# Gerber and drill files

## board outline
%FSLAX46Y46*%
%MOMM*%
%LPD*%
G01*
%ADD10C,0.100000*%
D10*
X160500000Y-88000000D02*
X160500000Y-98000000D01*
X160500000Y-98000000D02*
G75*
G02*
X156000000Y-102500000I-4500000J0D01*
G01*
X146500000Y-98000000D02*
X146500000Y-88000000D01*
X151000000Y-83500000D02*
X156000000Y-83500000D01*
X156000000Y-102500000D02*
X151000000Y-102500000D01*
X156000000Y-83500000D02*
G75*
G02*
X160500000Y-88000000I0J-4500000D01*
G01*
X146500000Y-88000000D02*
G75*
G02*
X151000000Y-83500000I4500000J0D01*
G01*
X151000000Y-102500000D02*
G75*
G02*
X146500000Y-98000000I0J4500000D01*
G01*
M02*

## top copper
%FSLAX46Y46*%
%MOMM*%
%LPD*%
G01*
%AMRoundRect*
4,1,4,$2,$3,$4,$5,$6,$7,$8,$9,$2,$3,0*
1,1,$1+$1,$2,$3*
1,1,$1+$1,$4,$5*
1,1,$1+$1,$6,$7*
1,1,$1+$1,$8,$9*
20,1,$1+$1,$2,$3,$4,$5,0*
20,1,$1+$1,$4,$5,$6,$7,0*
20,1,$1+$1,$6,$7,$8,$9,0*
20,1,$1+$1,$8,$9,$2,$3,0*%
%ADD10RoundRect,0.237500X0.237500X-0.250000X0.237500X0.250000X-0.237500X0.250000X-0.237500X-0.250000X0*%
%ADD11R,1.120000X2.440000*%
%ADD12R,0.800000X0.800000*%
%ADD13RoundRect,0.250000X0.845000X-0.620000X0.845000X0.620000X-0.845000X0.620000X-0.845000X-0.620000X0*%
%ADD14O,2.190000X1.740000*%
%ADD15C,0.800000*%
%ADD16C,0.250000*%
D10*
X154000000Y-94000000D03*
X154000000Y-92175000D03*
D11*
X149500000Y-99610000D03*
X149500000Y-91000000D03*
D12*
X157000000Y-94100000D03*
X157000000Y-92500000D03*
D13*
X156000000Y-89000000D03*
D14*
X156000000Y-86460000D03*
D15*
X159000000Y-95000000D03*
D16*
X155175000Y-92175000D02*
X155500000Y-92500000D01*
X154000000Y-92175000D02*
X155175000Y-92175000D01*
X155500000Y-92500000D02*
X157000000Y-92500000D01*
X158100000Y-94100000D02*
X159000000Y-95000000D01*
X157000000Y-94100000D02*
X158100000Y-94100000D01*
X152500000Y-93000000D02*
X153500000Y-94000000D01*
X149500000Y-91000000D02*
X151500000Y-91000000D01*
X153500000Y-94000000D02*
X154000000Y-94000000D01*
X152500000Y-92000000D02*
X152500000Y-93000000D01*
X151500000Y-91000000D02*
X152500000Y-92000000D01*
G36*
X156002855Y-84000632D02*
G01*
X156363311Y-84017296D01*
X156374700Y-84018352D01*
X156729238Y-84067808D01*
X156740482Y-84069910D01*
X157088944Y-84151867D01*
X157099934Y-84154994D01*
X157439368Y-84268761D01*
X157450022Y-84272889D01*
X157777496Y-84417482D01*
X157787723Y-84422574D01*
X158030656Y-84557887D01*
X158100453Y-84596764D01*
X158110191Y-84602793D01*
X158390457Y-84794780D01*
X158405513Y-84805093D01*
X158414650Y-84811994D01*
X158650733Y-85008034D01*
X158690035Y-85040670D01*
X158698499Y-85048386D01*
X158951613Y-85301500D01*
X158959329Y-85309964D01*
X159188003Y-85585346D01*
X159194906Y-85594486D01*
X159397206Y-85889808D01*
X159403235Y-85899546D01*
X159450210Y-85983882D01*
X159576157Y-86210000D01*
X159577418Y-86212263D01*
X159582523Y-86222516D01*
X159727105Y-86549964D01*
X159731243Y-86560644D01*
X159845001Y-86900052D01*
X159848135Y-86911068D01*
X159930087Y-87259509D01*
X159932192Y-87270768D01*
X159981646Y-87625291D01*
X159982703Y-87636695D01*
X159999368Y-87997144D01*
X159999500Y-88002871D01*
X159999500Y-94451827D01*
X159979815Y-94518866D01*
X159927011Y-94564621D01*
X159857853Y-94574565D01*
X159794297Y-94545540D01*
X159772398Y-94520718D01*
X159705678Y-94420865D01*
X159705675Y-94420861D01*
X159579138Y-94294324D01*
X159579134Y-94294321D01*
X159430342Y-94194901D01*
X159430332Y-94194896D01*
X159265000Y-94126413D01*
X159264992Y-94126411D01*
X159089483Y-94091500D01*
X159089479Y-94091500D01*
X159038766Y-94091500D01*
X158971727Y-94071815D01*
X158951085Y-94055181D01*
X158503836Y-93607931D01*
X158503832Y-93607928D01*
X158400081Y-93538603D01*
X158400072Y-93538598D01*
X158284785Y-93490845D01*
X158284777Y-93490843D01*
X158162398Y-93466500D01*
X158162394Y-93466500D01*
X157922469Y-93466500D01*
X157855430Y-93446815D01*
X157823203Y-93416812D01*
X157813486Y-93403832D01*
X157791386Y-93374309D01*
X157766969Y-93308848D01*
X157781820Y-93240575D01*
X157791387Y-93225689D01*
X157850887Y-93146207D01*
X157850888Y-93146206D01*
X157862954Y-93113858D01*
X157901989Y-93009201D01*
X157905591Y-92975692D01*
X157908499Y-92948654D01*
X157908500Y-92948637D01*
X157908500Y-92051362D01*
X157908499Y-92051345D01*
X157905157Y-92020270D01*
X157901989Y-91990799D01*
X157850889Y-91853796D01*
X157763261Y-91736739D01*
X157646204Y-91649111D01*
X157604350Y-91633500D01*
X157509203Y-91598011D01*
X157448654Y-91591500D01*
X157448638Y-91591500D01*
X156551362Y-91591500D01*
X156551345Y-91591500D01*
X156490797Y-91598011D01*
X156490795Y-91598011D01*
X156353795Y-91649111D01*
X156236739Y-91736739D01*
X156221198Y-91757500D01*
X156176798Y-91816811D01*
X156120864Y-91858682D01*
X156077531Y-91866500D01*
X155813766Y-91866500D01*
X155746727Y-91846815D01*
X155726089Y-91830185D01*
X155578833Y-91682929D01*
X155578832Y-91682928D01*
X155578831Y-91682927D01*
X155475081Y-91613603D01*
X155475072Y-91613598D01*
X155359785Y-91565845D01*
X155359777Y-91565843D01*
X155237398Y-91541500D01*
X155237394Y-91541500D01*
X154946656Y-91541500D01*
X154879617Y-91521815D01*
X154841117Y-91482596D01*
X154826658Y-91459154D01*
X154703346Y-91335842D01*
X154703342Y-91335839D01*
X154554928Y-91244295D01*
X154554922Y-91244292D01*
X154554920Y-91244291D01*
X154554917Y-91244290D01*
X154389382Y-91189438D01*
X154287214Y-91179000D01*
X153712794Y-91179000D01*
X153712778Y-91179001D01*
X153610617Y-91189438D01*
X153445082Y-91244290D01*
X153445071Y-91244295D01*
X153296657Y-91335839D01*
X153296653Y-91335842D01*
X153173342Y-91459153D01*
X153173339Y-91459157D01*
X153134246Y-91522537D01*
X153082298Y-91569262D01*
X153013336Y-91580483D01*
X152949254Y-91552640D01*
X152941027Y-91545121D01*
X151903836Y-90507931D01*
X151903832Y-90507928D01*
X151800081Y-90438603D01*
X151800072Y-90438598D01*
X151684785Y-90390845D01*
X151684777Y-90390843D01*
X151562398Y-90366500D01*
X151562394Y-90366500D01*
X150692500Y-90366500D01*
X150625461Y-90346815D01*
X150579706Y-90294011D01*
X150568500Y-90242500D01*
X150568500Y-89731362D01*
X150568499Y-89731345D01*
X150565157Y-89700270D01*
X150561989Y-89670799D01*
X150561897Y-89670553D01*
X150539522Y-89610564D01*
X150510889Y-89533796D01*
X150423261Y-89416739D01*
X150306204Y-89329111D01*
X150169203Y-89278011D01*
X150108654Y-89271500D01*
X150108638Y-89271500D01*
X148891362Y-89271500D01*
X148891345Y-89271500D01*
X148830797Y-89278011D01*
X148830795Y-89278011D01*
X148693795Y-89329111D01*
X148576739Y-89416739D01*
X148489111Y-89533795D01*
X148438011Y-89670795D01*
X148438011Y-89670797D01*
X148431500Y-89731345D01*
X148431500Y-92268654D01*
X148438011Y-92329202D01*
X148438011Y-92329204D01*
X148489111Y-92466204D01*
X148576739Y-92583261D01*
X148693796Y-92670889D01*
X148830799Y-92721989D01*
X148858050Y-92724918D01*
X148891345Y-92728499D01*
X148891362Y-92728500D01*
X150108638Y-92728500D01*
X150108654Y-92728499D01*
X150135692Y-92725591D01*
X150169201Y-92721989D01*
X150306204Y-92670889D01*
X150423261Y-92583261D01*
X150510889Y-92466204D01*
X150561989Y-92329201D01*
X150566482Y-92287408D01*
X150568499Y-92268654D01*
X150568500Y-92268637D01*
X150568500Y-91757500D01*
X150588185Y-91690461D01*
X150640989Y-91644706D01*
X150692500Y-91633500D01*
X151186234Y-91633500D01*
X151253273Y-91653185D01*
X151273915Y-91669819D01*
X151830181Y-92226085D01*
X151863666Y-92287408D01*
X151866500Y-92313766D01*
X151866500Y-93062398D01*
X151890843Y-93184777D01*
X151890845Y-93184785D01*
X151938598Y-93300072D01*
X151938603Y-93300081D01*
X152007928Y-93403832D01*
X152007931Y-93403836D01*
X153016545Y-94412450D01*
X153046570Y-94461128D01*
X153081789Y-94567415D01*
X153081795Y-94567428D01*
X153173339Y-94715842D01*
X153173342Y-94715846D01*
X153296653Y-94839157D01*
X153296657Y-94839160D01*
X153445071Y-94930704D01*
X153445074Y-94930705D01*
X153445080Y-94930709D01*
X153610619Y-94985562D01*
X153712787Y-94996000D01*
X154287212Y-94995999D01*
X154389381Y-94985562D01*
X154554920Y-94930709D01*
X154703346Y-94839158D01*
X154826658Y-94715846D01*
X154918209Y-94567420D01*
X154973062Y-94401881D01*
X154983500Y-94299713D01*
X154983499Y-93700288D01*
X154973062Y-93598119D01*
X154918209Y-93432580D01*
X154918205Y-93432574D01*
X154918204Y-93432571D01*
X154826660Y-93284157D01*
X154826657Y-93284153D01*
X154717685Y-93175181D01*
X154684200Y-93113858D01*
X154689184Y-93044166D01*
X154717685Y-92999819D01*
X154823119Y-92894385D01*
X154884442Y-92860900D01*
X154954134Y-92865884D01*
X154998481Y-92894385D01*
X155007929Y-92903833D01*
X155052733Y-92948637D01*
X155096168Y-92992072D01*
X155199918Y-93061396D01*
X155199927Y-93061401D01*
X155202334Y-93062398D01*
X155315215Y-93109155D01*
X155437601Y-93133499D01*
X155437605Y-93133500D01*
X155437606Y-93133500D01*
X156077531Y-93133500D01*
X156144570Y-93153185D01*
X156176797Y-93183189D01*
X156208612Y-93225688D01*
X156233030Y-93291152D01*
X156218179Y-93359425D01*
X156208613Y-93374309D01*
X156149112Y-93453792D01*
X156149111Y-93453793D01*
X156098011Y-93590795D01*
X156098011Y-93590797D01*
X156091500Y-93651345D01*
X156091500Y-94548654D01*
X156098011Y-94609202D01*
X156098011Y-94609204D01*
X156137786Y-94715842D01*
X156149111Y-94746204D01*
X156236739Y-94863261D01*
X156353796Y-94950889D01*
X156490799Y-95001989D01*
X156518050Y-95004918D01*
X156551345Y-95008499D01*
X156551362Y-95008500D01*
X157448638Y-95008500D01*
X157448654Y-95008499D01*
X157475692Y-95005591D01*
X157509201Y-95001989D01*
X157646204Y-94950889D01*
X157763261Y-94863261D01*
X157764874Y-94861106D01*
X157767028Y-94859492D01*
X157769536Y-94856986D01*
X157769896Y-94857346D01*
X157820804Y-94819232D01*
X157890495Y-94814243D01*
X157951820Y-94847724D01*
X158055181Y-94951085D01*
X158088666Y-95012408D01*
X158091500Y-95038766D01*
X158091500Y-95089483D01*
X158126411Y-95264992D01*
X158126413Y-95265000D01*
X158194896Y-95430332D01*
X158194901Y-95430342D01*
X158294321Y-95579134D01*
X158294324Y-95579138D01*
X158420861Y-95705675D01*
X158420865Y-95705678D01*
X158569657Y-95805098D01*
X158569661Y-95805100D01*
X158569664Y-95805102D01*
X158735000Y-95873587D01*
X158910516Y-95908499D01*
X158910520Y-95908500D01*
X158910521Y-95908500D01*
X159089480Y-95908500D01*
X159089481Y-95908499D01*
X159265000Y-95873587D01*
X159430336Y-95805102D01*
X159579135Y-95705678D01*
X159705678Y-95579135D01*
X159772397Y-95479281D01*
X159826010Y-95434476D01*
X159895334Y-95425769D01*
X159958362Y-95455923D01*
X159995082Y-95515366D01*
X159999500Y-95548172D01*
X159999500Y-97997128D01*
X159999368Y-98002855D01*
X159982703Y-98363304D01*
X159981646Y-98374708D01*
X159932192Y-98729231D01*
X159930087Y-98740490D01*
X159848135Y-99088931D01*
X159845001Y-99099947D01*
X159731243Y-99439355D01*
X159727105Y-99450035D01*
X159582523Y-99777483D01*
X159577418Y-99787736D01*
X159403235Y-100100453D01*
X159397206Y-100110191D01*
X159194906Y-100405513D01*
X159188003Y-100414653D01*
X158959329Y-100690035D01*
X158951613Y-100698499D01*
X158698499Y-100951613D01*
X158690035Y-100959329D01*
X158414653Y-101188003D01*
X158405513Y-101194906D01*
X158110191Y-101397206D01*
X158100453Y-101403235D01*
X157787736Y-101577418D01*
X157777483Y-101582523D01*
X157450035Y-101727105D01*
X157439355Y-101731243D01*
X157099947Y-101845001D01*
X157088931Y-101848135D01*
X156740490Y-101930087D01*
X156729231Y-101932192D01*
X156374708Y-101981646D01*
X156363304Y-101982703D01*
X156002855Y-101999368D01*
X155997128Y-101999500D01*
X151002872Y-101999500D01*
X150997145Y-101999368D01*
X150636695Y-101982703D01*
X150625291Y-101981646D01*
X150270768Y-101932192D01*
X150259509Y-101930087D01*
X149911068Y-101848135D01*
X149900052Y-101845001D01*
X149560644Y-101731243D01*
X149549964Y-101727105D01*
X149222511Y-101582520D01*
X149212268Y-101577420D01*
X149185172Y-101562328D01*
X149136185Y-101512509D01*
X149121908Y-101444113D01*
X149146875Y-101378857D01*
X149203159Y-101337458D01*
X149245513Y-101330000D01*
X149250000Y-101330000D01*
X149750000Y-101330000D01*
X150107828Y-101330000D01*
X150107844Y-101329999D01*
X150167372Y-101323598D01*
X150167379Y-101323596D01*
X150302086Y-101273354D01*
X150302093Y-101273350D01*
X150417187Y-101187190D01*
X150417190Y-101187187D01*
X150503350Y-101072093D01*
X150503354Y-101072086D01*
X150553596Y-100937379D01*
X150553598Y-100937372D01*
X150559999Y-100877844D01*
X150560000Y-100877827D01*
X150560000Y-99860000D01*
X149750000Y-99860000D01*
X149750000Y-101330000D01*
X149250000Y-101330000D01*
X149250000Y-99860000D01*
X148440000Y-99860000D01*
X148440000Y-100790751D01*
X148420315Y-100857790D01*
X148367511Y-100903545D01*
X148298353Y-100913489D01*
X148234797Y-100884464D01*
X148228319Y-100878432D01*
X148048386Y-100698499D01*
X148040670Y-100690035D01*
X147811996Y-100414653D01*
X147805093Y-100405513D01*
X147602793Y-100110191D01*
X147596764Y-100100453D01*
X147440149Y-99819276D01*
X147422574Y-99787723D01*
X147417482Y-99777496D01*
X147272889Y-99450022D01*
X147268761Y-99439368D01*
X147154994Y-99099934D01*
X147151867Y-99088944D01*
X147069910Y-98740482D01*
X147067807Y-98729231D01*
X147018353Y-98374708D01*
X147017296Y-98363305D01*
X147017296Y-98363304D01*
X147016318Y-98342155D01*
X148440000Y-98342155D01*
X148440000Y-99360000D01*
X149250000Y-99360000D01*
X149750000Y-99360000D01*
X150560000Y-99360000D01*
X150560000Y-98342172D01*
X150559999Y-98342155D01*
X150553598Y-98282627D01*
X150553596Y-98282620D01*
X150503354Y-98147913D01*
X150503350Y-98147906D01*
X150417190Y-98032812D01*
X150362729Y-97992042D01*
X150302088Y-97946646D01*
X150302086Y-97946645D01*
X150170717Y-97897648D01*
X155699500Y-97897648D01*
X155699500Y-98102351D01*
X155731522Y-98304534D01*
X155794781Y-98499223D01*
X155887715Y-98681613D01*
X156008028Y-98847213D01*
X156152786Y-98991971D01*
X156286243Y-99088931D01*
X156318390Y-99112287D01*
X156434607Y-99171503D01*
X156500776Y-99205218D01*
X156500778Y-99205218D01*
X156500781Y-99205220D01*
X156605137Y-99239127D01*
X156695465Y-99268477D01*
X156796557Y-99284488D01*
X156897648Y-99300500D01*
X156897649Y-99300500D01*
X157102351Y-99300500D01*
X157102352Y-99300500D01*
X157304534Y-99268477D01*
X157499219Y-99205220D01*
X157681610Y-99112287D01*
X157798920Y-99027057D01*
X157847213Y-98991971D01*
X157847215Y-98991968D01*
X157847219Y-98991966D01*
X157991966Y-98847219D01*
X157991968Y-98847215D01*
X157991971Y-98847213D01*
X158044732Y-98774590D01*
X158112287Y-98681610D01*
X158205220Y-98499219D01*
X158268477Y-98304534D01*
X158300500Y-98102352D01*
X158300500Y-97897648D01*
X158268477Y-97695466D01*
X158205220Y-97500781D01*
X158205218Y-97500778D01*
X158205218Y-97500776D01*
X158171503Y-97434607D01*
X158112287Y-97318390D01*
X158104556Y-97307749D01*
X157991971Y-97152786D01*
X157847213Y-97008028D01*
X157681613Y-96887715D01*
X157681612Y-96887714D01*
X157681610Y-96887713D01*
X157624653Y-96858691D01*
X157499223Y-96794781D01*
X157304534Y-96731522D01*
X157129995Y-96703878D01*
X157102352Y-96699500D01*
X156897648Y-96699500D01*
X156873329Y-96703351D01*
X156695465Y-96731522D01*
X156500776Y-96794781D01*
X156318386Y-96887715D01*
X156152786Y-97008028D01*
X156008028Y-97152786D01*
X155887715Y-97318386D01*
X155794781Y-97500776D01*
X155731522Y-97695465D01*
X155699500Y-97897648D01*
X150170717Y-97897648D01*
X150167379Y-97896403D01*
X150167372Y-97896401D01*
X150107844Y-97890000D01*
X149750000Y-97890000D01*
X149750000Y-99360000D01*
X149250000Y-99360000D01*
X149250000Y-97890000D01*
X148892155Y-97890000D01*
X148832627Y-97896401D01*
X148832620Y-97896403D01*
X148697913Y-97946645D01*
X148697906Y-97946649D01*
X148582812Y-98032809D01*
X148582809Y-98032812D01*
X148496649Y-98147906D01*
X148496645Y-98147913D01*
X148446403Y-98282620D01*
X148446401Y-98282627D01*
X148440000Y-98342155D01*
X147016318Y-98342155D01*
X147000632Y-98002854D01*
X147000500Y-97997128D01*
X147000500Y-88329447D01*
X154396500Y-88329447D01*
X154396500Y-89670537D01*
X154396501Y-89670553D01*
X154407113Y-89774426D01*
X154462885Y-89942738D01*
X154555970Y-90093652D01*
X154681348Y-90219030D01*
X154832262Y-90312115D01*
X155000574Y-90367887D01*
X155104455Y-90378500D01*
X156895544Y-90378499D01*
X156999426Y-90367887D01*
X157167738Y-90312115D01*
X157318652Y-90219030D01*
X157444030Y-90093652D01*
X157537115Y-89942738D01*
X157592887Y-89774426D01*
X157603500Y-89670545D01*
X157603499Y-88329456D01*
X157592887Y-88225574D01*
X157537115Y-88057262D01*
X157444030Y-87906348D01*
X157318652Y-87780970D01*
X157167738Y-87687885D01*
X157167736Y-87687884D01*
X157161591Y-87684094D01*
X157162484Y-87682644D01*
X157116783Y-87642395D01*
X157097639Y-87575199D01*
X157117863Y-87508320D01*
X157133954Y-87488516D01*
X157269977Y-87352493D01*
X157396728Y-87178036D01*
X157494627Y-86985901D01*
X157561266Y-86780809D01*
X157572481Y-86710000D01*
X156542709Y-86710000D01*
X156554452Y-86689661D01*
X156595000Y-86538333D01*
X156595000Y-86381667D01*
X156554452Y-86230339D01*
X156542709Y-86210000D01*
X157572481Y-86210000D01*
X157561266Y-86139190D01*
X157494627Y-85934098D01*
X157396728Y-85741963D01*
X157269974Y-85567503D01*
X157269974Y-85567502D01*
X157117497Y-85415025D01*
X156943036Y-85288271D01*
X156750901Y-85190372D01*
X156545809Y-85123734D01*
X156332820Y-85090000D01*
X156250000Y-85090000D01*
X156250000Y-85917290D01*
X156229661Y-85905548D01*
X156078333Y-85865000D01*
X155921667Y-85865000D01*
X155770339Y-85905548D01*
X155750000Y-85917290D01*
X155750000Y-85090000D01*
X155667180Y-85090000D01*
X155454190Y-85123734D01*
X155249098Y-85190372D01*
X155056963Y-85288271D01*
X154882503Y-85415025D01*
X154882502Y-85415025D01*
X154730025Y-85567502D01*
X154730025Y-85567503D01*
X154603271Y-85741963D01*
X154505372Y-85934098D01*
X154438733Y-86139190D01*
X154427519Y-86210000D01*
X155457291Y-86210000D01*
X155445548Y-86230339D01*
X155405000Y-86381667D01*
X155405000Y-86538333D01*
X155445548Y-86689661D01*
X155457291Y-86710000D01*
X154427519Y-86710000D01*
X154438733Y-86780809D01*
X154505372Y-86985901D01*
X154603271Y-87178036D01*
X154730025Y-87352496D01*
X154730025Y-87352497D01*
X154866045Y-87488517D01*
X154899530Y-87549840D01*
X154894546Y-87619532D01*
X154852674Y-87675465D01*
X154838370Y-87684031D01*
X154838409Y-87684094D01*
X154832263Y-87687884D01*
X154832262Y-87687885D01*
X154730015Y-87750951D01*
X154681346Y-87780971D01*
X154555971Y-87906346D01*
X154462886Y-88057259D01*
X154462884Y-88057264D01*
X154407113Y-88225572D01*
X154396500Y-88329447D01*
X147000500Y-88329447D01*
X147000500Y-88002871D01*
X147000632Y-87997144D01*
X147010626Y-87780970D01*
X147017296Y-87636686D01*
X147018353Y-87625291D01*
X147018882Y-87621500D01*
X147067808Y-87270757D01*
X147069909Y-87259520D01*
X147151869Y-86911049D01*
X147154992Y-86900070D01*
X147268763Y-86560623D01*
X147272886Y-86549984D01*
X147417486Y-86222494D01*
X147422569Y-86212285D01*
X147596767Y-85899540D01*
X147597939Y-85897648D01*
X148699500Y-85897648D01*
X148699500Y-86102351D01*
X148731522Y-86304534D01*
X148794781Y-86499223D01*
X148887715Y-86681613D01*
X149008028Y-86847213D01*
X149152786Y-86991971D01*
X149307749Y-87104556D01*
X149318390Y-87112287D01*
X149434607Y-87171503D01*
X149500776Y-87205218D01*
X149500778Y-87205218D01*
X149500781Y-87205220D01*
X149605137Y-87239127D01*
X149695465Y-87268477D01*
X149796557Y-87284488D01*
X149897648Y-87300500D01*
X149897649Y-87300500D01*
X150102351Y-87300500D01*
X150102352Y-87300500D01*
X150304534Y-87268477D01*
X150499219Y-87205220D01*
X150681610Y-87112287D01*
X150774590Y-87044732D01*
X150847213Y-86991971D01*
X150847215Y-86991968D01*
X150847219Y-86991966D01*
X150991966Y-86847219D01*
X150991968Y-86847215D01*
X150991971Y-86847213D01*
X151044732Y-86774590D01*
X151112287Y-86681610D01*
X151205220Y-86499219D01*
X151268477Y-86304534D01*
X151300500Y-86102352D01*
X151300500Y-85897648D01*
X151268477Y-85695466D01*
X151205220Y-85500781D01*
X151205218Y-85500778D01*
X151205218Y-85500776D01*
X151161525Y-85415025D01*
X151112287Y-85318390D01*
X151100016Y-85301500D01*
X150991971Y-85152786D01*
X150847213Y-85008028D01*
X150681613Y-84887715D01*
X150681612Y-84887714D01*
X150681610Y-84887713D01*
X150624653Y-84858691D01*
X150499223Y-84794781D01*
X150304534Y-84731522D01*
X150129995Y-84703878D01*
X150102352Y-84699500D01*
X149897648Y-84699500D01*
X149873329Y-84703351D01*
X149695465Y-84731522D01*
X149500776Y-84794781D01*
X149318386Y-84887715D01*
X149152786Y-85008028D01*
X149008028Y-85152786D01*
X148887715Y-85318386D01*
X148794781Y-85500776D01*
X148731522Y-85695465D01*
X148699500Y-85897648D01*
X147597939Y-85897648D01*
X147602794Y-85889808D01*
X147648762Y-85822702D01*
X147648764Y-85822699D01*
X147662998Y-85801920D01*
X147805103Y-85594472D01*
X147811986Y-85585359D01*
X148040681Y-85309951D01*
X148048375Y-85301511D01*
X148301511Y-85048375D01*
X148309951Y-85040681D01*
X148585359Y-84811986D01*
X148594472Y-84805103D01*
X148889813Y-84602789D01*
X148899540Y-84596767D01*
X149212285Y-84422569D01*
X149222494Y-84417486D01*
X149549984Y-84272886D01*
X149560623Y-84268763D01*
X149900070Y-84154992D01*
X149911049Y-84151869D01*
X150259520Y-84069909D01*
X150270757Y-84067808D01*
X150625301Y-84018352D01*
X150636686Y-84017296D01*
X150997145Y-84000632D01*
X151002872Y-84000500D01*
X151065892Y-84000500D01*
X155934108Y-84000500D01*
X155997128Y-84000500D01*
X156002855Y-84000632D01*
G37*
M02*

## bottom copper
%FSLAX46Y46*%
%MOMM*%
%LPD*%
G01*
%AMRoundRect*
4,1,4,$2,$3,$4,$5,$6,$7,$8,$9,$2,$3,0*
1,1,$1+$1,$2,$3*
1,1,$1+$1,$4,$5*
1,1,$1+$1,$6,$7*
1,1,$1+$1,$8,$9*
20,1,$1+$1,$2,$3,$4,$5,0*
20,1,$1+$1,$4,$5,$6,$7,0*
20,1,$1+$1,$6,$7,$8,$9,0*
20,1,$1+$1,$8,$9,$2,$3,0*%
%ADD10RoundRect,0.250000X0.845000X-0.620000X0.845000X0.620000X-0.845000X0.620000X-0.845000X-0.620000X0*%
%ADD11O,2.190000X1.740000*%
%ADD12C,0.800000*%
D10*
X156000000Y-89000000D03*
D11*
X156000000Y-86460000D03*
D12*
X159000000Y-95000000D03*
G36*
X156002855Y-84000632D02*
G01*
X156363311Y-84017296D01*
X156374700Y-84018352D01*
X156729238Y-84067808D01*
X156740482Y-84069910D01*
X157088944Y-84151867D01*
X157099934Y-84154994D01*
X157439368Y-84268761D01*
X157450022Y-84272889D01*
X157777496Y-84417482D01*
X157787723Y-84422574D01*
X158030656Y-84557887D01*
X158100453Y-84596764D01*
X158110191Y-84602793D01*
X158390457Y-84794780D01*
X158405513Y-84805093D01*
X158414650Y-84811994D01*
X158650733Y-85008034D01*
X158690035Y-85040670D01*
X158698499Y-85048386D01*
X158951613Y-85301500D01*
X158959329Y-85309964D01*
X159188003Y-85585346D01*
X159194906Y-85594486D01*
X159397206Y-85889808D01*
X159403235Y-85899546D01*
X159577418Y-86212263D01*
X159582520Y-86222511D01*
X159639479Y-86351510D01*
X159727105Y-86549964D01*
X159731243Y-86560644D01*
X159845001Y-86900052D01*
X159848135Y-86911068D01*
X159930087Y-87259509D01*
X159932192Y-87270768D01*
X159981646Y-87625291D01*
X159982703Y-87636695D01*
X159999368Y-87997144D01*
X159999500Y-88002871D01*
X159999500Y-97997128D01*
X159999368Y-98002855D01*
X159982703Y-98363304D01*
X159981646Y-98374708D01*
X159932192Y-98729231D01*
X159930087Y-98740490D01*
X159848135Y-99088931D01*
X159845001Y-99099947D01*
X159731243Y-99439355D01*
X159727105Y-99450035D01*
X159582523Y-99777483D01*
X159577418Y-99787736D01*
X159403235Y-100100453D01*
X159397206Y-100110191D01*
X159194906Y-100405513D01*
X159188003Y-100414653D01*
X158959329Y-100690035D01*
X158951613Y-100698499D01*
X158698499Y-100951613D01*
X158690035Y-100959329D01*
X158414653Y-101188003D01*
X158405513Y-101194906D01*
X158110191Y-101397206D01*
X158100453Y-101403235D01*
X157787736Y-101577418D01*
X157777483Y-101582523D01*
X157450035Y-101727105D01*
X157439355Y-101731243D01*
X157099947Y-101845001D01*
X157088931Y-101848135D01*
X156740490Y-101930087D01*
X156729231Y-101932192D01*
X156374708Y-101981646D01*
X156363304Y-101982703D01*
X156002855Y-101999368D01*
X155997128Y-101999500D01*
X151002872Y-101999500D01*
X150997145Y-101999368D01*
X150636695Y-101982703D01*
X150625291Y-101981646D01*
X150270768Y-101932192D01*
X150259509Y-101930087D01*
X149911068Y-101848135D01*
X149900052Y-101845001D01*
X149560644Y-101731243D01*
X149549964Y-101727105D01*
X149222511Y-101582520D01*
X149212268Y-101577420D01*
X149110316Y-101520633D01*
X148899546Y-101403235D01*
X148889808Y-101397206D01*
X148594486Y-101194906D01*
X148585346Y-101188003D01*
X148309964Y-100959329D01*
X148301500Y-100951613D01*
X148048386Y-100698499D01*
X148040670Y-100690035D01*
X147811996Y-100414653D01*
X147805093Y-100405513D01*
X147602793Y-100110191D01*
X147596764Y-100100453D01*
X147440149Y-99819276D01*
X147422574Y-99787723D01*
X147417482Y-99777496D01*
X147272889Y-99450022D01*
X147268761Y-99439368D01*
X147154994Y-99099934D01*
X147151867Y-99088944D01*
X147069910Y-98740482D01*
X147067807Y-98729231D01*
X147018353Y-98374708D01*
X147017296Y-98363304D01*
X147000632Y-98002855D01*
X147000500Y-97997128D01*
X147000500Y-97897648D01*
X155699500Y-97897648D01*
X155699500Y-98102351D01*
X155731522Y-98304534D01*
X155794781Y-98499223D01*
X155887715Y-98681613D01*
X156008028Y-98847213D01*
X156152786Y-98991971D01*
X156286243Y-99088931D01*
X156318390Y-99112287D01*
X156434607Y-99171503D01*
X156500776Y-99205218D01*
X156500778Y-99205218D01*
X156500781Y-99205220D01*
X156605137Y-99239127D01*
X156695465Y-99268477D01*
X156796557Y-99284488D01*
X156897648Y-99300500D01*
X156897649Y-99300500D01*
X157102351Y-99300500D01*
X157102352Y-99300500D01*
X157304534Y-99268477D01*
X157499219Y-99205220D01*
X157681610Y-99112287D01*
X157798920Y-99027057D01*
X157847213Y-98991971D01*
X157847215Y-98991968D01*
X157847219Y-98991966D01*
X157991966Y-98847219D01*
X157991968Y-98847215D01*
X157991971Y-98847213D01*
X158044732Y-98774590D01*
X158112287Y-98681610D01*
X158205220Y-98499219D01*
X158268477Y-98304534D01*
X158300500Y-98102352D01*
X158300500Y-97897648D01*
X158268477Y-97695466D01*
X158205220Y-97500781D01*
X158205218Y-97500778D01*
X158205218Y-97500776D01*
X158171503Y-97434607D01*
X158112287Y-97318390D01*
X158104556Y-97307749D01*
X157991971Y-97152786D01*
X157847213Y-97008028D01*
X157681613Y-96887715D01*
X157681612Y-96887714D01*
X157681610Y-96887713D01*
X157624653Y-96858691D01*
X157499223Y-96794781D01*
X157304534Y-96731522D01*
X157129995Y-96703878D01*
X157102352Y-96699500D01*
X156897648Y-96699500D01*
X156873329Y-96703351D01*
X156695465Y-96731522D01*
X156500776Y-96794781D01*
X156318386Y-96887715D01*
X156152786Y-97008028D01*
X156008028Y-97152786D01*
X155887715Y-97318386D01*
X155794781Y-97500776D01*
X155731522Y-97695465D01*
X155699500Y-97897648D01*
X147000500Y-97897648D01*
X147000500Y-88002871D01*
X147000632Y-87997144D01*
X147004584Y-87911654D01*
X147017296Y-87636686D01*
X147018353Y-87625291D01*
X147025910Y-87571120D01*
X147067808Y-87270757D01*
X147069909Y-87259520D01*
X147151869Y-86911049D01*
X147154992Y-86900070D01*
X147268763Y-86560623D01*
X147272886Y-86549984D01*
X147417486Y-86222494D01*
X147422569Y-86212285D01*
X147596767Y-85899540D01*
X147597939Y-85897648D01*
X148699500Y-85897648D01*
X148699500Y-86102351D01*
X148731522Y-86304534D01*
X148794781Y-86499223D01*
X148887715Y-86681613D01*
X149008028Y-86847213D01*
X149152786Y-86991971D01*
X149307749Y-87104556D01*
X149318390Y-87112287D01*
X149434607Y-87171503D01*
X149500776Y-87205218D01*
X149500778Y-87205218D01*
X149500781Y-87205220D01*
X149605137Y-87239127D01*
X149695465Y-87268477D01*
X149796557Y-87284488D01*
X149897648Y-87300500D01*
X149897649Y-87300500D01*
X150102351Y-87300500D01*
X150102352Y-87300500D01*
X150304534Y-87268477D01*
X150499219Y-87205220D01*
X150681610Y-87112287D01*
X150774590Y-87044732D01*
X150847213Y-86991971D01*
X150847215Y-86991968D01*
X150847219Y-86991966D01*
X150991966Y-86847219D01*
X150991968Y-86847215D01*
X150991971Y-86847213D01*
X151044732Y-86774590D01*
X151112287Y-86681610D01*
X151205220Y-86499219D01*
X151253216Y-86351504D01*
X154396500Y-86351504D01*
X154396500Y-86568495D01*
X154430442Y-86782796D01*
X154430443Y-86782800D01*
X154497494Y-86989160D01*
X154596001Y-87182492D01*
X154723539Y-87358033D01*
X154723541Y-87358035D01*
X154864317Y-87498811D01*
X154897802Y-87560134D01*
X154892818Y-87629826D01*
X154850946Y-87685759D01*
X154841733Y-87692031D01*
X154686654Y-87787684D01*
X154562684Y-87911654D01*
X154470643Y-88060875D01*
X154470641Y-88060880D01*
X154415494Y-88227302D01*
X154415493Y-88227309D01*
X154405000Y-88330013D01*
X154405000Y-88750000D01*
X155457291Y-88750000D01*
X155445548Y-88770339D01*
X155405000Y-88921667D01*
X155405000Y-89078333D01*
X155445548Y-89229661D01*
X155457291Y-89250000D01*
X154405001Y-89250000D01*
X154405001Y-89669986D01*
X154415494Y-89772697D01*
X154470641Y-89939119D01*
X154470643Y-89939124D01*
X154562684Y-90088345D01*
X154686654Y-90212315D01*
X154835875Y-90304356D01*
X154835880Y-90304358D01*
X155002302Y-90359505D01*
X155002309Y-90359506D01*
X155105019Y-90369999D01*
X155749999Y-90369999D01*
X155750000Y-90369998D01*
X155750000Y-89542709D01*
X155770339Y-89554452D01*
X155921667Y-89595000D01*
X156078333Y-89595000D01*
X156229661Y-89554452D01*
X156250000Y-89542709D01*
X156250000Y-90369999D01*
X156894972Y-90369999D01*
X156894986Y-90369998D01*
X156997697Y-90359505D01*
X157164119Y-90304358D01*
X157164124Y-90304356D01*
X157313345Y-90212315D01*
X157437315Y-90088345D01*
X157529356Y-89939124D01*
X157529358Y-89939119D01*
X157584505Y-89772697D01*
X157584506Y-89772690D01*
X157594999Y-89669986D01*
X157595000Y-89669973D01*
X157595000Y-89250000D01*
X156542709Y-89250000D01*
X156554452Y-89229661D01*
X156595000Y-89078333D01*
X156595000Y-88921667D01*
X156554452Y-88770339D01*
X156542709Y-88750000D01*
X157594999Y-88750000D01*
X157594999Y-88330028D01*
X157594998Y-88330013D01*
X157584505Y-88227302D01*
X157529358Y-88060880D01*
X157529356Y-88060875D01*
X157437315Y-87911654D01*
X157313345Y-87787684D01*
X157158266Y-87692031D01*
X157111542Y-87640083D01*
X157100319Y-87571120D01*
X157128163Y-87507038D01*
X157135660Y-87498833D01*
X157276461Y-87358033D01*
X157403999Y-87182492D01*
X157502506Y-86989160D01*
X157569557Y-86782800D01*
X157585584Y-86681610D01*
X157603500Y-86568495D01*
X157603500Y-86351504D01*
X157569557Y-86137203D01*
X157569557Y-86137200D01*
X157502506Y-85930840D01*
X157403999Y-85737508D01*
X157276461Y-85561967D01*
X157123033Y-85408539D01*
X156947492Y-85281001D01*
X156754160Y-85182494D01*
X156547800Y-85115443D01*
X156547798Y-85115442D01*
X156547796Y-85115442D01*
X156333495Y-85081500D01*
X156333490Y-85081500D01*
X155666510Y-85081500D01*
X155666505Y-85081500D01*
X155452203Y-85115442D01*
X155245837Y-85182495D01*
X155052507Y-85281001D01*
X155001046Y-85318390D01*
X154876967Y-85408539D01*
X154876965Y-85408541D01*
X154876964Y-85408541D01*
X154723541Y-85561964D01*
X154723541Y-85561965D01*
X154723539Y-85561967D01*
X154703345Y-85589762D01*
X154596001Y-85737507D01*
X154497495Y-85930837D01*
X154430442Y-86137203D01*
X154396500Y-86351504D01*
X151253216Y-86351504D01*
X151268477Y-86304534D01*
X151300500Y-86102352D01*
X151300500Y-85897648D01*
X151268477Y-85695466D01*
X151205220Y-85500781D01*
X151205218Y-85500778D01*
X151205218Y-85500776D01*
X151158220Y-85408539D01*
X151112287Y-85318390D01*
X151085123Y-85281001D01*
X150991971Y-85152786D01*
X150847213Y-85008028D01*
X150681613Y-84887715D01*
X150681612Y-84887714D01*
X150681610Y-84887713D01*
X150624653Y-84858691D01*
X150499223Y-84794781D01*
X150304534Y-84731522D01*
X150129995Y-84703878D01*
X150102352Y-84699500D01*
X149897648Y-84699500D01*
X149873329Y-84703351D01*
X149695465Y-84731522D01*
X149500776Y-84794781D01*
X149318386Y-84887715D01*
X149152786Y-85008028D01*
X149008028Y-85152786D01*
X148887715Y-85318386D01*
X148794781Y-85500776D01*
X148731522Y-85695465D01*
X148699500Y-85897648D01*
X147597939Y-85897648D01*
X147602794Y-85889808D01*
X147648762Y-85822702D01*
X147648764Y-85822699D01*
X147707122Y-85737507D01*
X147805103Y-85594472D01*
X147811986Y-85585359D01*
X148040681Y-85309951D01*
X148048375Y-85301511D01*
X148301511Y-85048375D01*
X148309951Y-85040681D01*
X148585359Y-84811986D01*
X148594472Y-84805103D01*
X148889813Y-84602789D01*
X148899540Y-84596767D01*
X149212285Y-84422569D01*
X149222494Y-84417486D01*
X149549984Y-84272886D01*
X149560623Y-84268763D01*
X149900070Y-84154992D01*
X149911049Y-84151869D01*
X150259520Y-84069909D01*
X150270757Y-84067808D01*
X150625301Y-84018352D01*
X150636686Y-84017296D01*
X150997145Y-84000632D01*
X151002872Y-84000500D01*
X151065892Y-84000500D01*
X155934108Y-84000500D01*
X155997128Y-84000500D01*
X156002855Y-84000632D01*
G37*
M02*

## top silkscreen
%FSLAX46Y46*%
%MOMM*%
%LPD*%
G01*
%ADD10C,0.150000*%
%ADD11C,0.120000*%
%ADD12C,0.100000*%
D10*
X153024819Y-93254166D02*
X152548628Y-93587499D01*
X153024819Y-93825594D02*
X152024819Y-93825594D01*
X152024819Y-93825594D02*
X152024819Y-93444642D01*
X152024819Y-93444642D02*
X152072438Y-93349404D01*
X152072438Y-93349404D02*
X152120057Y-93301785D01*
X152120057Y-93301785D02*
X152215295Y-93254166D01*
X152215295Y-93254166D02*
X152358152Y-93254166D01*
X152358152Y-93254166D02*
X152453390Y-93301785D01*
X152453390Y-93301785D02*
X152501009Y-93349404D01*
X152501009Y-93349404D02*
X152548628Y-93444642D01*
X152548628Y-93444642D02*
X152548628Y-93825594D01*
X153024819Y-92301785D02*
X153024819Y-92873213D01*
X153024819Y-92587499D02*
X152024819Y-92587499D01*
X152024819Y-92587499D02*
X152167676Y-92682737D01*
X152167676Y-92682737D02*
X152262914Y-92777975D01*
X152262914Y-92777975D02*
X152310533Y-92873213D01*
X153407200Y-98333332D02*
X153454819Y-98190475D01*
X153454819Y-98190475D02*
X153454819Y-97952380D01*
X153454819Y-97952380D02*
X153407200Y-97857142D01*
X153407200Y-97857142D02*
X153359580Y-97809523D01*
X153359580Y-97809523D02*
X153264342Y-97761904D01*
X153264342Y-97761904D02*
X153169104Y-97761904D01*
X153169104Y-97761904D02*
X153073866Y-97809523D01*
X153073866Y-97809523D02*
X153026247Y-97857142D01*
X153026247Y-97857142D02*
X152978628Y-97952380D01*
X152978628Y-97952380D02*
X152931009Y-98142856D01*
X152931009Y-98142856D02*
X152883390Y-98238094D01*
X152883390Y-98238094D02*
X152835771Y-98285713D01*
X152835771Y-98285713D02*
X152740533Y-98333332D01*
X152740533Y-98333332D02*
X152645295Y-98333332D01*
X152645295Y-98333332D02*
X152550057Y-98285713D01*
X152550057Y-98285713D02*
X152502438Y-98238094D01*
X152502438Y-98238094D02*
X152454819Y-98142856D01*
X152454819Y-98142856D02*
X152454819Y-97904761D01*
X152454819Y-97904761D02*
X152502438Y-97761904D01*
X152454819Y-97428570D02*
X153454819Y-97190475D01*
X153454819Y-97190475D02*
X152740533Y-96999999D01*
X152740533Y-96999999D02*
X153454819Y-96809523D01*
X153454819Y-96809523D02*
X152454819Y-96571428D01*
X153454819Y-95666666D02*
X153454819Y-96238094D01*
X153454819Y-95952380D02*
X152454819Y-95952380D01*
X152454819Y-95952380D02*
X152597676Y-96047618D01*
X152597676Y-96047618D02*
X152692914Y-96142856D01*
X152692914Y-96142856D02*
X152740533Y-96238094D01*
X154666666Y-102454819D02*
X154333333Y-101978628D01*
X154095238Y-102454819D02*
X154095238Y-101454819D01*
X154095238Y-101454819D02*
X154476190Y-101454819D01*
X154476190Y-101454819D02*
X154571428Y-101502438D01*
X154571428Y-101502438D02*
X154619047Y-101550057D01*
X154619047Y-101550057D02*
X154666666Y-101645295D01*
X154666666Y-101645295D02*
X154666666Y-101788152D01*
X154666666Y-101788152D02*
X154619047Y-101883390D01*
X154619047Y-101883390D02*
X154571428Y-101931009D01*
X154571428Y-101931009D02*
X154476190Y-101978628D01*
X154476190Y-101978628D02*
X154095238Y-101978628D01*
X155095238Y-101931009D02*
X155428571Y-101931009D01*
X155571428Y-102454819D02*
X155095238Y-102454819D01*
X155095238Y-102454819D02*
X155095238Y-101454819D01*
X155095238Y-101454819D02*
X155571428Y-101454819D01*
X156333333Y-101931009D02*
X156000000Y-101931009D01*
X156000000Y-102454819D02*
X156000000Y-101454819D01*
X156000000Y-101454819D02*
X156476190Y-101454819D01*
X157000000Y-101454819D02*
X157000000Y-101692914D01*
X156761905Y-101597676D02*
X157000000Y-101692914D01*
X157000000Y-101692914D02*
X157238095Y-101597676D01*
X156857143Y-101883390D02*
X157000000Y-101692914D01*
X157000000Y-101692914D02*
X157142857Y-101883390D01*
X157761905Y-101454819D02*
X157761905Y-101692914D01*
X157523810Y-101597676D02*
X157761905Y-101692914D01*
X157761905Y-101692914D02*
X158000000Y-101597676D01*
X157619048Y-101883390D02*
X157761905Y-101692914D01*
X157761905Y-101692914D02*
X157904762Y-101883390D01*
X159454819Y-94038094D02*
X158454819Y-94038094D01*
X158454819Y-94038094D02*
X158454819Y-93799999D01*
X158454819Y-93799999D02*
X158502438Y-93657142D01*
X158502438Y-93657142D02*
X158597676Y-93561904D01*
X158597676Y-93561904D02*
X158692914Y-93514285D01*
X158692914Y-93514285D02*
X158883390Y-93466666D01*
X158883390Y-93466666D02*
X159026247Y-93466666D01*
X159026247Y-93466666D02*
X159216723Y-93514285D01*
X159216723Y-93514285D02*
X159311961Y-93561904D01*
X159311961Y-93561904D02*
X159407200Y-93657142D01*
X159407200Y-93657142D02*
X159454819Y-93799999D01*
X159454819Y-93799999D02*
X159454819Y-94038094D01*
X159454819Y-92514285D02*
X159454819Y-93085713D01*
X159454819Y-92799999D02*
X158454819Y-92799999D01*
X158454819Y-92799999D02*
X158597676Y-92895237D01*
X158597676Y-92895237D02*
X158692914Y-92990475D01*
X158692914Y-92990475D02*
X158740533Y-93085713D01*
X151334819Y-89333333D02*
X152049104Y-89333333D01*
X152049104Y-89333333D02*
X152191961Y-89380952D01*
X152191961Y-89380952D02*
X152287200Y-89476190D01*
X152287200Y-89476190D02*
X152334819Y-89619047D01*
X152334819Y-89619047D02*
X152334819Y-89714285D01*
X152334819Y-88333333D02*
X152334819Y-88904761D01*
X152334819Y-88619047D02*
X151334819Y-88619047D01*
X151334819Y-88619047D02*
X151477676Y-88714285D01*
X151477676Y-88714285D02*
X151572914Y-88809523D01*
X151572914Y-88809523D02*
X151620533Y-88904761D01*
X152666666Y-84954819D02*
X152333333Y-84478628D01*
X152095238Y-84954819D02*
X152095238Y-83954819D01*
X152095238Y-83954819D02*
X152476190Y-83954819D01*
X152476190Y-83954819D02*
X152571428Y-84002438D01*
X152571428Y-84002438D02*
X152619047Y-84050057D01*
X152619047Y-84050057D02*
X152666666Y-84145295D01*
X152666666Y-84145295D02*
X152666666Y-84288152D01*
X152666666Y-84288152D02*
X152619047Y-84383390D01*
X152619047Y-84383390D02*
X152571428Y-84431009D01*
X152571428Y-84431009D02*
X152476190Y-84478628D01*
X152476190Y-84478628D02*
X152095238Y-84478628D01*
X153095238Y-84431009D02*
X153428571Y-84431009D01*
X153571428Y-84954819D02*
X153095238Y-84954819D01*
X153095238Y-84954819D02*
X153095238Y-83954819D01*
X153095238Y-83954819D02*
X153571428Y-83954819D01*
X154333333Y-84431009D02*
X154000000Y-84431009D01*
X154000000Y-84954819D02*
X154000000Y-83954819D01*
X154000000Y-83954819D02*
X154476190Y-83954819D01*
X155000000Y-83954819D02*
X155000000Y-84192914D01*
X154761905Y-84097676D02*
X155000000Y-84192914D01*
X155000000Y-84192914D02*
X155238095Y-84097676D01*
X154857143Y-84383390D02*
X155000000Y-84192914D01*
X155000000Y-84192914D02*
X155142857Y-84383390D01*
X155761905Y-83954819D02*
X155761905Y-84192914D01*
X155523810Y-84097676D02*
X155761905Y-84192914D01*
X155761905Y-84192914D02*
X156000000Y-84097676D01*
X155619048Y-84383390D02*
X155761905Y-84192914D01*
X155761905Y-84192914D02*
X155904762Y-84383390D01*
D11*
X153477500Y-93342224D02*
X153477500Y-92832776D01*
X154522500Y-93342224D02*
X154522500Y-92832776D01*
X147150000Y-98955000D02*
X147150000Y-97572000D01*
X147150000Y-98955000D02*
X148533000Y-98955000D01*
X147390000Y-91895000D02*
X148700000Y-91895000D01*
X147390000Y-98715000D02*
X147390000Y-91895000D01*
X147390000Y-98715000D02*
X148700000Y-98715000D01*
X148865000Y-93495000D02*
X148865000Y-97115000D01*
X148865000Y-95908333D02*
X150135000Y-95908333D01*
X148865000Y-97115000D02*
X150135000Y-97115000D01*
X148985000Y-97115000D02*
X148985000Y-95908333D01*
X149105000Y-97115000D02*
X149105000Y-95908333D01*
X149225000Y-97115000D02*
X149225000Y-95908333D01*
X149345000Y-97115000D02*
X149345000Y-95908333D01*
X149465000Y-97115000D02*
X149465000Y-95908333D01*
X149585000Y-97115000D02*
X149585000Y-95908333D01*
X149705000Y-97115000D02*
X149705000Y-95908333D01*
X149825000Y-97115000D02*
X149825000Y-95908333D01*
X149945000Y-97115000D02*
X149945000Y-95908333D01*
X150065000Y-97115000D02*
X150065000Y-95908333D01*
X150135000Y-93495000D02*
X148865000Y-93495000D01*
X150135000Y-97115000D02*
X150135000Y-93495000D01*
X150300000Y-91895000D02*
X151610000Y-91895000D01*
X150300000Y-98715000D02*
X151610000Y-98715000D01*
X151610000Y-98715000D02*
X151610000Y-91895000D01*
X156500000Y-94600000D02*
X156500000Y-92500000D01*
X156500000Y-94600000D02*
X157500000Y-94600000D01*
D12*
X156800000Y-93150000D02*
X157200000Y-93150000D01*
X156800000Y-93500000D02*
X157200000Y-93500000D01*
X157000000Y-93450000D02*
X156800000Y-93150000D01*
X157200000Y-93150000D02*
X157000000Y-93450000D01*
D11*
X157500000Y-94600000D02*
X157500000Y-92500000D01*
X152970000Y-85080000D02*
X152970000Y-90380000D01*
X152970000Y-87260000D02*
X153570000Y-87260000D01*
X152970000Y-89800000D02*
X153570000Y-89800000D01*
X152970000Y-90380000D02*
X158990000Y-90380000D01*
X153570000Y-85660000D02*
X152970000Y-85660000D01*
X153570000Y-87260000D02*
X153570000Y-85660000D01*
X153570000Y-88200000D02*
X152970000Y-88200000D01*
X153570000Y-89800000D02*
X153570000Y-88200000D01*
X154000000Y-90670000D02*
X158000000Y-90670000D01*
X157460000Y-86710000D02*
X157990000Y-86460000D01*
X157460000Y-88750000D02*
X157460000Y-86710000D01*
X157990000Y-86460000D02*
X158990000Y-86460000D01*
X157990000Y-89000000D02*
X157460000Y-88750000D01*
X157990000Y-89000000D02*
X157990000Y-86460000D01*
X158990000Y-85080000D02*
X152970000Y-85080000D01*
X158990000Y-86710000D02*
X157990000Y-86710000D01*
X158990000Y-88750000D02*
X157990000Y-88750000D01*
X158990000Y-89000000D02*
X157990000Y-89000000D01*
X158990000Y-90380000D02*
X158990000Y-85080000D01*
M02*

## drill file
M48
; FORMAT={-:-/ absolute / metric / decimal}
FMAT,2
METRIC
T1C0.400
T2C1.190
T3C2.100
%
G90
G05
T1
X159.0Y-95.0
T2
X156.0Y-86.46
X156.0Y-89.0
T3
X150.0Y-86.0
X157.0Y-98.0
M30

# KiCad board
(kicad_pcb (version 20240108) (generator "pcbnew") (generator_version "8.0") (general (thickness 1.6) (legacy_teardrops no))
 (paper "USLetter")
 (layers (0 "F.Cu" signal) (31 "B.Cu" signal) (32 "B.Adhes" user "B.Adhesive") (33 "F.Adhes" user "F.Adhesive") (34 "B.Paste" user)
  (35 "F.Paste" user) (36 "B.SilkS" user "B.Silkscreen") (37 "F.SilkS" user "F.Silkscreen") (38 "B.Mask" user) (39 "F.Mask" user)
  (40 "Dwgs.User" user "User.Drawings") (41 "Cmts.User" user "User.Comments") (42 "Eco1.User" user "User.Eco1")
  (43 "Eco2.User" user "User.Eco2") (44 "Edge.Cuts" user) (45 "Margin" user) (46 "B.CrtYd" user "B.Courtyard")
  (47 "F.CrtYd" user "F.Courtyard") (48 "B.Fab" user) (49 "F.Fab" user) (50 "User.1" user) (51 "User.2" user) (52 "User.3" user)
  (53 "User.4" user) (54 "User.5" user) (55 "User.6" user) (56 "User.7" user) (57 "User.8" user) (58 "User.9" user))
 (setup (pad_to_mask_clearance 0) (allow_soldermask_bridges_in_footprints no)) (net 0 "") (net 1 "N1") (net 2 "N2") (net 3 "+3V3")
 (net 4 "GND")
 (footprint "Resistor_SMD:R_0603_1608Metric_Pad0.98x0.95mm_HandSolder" (layer "F.Cu") (at 154 93.0875 90)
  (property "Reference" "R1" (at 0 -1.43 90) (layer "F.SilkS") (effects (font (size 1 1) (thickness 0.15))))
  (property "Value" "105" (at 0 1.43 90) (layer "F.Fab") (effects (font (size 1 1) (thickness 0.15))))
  (fp_line (start -0.254724 -0.5225) (end 0.254724 -0.5225) (stroke (width 0.12) (type solid)) (layer "F.SilkS"))
  (fp_line (start -0.254724 0.5225) (end 0.254724 0.5225) (stroke (width 0.12) (type solid)) (layer "F.SilkS"))
  (pad "1" smd roundrect (at -0.9125 0 90) (size 0.975 0.95) (layers "F.Cu" "F.Paste" "F.Mask") (roundrect_rratio 0.25) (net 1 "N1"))
  (pad "2" smd roundrect (at 0.9125 0 90) (size 0.975 0.95) (layers "F.Cu" "F.Paste" "F.Mask") (roundrect_rratio 0.25) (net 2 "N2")))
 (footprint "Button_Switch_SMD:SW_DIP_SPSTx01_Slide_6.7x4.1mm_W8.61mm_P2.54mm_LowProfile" (layer "F.Cu") (at 149.5 95.305 90)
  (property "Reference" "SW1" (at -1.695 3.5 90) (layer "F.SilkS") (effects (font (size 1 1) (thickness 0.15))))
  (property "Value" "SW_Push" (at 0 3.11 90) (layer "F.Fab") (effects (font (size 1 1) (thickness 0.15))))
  (fp_line (start -3.65 -2.35) (end -2.267 -2.35) (stroke (width 0.12) (type solid)) (layer "F.SilkS"))
  (fp_line (start -3.65 -2.35) (end -3.65 -0.967) (stroke (width 0.12) (type solid)) (layer "F.SilkS"))
  (fp_line (start 3.41 -2.11) (end 3.41 -0.8) (stroke (width 0.12) (type solid)) (layer "F.SilkS"))
  (fp_line (start -3.41 -2.11) (end 3.41 -2.11) (stroke (width 0.12) (type solid)) (layer "F.SilkS"))
  (fp_line (start -3.41 -2.11) (end -3.41 -0.8) (stroke (width 0.12) (type solid)) (layer "F.SilkS"))
  (fp_line (start 1.81 -0.635) (end -1.81 -0.635) (stroke (width 0.12) (type solid)) (layer "F.SilkS"))
  (fp_line (start -0.603333 -0.635) (end -0.603333 0.635) (stroke (width 0.12) (type solid)) (layer "F.SilkS"))
  (fp_line (start -1.81 -0.635) (end -1.81 0.635) (stroke (width 0.12) (type solid)) (layer "F.SilkS"))
  (fp_line (start -1.81 -0.515) (end -0.603333 -0.515) (stroke (width 0.12) (type solid)) (layer "F.SilkS"))
  (fp_line (start -1.81 -0.395) (end -0.603333 -0.395) (stroke (width 0.12) (type solid)) (layer "F.SilkS"))
  (fp_line (start -1.81 -0.275) (end -0.603333 -0.275) (stroke (width 0.12) (type solid)) (layer "F.SilkS"))
  (fp_line (start -1.81 -0.155) (end -0.603333 -0.155) (stroke (width 0.12) (type solid)) (layer "F.SilkS"))
  (fp_line (start -1.81 -0.035) (end -0.603333 -0.035) (stroke (width 0.12) (type solid)) (layer "F.SilkS"))
  (fp_line (start -1.81 0.085) (end -0.603333 0.085) (stroke (width 0.12) (type solid)) (layer "F.SilkS"))
  (fp_line (start -1.81 0.205) (end -0.603333 0.205) (stroke (width 0.12) (type solid)) (layer "F.SilkS"))
  (fp_line (start -1.81 0.325) (end -0.603333 0.325) (stroke (width 0.12) (type solid)) (layer "F.SilkS"))
  (fp_line (start -1.81 0.445) (end -0.603333 0.445) (stroke (width 0.12) (type solid)) (layer "F.SilkS"))
  (fp_line (start -1.81 0.565) (end -0.603333 0.565) (stroke (width 0.12) (type solid)) (layer "F.SilkS"))
  (fp_line (start 1.81 0.635) (end 1.81 -0.635) (stroke (width 0.12) (type solid)) (layer "F.SilkS"))
  (fp_line (start -1.81 0.635) (end 1.81 0.635) (stroke (width 0.12) (type solid)) (layer "F.SilkS"))
  (fp_line (start 3.41 0.8) (end 3.41 2.11) (stroke (width 0.12) (type solid)) (layer "F.SilkS"))
  (fp_line (start -3.41 0.8) (end -3.41 2.11) (stroke (width 0.12) (type solid)) (layer "F.SilkS"))
  (fp_line (start -3.41 2.11) (end 3.41 2.11) (stroke (width 0.12) (type solid)) (layer "F.SilkS"))
  (pad "1" smd rect (at -4.305 0 90) (size 2.44 1.12) (layers "F.Cu" "F.Paste" "F.Mask") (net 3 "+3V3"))
  (pad "2" smd rect (at 4.305 0 90) (size 2.44 1.12) (layers "F.Cu" "F.Paste" "F.Mask") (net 1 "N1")))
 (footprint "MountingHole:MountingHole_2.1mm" (layer "F.Cu") (at 157 98)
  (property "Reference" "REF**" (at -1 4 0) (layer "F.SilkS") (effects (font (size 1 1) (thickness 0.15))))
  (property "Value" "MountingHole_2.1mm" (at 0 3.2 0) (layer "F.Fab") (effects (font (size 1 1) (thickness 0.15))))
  (pad "" np_thru_hole circle (at 0 0) (size 2.1 2.1) (drill 2.1) (layers "*.Cu" "*.Mask")))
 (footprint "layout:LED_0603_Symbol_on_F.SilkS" (layer "F.Cu") (at 157 93.3 90)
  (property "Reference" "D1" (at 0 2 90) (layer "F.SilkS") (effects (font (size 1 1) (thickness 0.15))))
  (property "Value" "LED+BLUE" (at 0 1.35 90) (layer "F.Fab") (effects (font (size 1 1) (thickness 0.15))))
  (fp_line (start -1.3 -0.5) (end 0.8 -0.5) (stroke (width 0.12) (type solid)) (layer "F.SilkS"))
  (fp_line (start -1.3 -0.5) (end -1.3 0.5) (stroke (width 0.12) (type solid)) (layer "F.SilkS"))
  (fp_line (start 0.15 -0.2) (end 0.15 0.2) (stroke (width 0.1) (type solid)) (layer "F.SilkS"))
  (fp_line (start -0.2 -0.2) (end -0.2 0.2) (stroke (width 0.1) (type solid)) (layer "F.SilkS"))
  (fp_line (start -0.15 0) (end 0.15 -0.2) (stroke (width 0.1) (type solid)) (layer "F.SilkS"))
  (fp_line (start 0.15 0.2) (end -0.15 0) (stroke (width 0.1) (type solid)) (layer "F.SilkS"))
  (fp_line (start -1.3 0.5) (end 0.8 0.5) (stroke (width 0.12) (type solid)) (layer "F.SilkS"))
  (pad "1" smd rect (at -0.8 0 270) (size 0.8 0.8) (layers "F.Cu" "F.Paste" "F.Mask") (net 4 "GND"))
  (pad "2" smd rect (at 0.8 0 270) (size 0.8 0.8) (layers "F.Cu" "F.Paste" "F.Mask") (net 2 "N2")))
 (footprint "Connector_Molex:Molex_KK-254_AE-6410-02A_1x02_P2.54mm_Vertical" (layer "F.Cu") (at 156 89 90)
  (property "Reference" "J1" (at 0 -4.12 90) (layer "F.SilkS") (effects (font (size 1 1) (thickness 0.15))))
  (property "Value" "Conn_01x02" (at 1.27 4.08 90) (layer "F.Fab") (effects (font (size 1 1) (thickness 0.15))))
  (fp_line (start 3.92 -3.03) (end -1.38 -3.03) (stroke (width 0.12) (type solid)) (layer "F.SilkS"))
  (fp_line (start 1.74 -3.03) (end 1.74 -2.43) (stroke (width 0.12) (type solid)) (layer "F.SilkS"))
  (fp_line (start -0.8 -3.03) (end -0.8 -2.43) (stroke (width 0.12) (type solid)) (layer "F.SilkS"))
  (fp_line (start -1.38 -3.03) (end -1.38 2.99) (stroke (width 0.12) (type solid)) (layer "F.SilkS"))
  (fp_line (start 3.34 -2.43) (end 3.34 -3.03) (stroke (width 0.12) (type solid)) (layer "F.SilkS"))
  (fp_line (start 1.74 -2.43) (end 3.34 -2.43) (stroke (width 0.12) (type solid)) (layer "F.SilkS"))
  (fp_line (start 0.8 -2.43) (end 0.8 -3.03) (stroke (width 0.12) (type solid)) (layer "F.SilkS"))
  (fp_line (start -0.8 -2.43) (end 0.8 -2.43) (stroke (width 0.12) (type solid)) (layer "F.SilkS"))
  (fp_line (start -1.67 -2) (end -1.67 2) (stroke (width 0.12) (type solid)) (layer "F.SilkS"))
  (fp_line (start 2.29 1.46) (end 2.54 1.99) (stroke (width 0.12) (type solid)) (layer "F.SilkS"))
  (fp_line (start 0.25 1.46) (end 2.29 1.46) (stroke (width 0.12) (type solid)) (layer "F.SilkS"))
  (fp_line (start 2.54 1.99) (end 2.54 2.99) (stroke (width 0.12) (type solid)) (layer "F.SilkS"))
  (fp_line (start 0 1.99) (end 0.25 1.46) (stroke (width 0.12) (type solid)) (layer "F.SilkS"))
  (fp_line (start 0 1.99) (end 2.54 1.99) (stroke (width 0.12) (type solid)) (layer "F.SilkS"))
  (fp_line (start 3.92 2.99) (end 3.92 -3.03) (stroke (width 0.12) (type solid)) (layer "F.SilkS"))
  (fp_line (start 2.29 2.99) (end 2.29 1.99) (stroke (width 0.12) (type solid)) (layer "F.SilkS"))
  (fp_line (start 0.25 2.99) (end 0.25 1.99) (stroke (width 0.12) (type solid)) (layer "F.SilkS"))
  (fp_line (start 0 2.99) (end 0 1.99) (stroke (width 0.12) (type solid)) (layer "F.SilkS"))
  (fp_line (start -1.38 2.99) (end 3.92 2.99) (stroke (width 0.12) (type solid)) (layer "F.SilkS"))
  (pad "1" thru_hole roundrect (at 0 0 90) (size 1.74 2.19) (drill 1.19) (layers "*.Cu" "*.Mask") (remove_unused_layers no)
   (roundrect_rratio 0.143678) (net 4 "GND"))
  (pad "2" thru_hole oval (at 2.54 0 90) (size 1.74 2.19) (drill 1.19) (layers "*.Cu" "*.Mask") (remove_unused_layers no) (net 3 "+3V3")))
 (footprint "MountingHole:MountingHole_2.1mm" (layer "F.Cu") (at 150 86)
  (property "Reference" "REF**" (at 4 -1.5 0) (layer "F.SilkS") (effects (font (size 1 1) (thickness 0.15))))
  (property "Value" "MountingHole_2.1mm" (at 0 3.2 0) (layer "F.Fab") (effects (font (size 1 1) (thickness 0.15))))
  (pad "" np_thru_hole circle (at 0 0) (size 2.1 2.1) (drill 2.1) (layers "*.Cu" "*.Mask")))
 (gr_line (start 160.5 88) (end 160.5 98) (stroke (width 0.1) (type default)) (layer "Edge.Cuts"))
 (gr_arc (start 160.5 98) (mid 159.181981 101.181981) (end 156 102.5) (stroke (width 0.1) (type default)) (layer "Edge.Cuts"))
 (gr_line (start 146.5 98) (end 146.5 88) (stroke (width 0.1) (type default)) (layer "Edge.Cuts"))
 (gr_line (start 151 83.5) (end 156 83.5) (stroke (width 0.1) (type default)) (layer "Edge.Cuts"))
 (gr_line (start 156 102.5) (end 151 102.5) (stroke (width 0.1) (type default)) (layer "Edge.Cuts"))
 (gr_arc (start 156 83.5) (mid 159.181981 84.818019) (end 160.5 88) (stroke (width 0.1) (type default)) (layer "Edge.Cuts"))
 (gr_arc (start 146.5 88) (mid 147.818019 84.818019) (end 151 83.5) (stroke (width 0.1) (type default)) (layer "Edge.Cuts"))
 (gr_arc (start 151 102.5) (mid 147.818019 101.181981) (end 146.5 98) (stroke (width 0.1) (type default)) (layer "Edge.Cuts"))
 (segment (start 155.175 92.175) (end 155.5 92.5) (width 0.25) (layer "F.Cu") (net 2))
 (segment (start 154 92.175) (end 155.175 92.175) (width 0.25) (layer "F.Cu") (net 2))
 (segment (start 155.5 92.5) (end 157 92.5) (width 0.25) (layer "F.Cu") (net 2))
 (segment (start 158.1 94.1) (end 159 95) (width 0.25) (layer "F.Cu") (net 4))
 (segment (start 157 94.1) (end 158.1 94.1) (width 0.25) (layer "F.Cu") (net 4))
 (via (at 159 95) (size 0.8) (drill 0.4) (layers "F.Cu" "B.Cu") (free yes) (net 4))
 (segment (start 152.5 93) (end 153.5 94) (width 0.25) (layer "F.Cu") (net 1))
 (segment (start 149.5 91) (end 151.5 91) (width 0.25) (layer "F.Cu") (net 1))
 (segment (start 153.5 94) (end 154 94) (width 0.25) (layer "F.Cu") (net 1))
 (segment (start 152.5 92) (end 152.5 93) (width 0.25) (layer "F.Cu") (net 1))
 (segment (start 151.5 91) (end 152.5 92) (width 0.25) (layer "F.Cu") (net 1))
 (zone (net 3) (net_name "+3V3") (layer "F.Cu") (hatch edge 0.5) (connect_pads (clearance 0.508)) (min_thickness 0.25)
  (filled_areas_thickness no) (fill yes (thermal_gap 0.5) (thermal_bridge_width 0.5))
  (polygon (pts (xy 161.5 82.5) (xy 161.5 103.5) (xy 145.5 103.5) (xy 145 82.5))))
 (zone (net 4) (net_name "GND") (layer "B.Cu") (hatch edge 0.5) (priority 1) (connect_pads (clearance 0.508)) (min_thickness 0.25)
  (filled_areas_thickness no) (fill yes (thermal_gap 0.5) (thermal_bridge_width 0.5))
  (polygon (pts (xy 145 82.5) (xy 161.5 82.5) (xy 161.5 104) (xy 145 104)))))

